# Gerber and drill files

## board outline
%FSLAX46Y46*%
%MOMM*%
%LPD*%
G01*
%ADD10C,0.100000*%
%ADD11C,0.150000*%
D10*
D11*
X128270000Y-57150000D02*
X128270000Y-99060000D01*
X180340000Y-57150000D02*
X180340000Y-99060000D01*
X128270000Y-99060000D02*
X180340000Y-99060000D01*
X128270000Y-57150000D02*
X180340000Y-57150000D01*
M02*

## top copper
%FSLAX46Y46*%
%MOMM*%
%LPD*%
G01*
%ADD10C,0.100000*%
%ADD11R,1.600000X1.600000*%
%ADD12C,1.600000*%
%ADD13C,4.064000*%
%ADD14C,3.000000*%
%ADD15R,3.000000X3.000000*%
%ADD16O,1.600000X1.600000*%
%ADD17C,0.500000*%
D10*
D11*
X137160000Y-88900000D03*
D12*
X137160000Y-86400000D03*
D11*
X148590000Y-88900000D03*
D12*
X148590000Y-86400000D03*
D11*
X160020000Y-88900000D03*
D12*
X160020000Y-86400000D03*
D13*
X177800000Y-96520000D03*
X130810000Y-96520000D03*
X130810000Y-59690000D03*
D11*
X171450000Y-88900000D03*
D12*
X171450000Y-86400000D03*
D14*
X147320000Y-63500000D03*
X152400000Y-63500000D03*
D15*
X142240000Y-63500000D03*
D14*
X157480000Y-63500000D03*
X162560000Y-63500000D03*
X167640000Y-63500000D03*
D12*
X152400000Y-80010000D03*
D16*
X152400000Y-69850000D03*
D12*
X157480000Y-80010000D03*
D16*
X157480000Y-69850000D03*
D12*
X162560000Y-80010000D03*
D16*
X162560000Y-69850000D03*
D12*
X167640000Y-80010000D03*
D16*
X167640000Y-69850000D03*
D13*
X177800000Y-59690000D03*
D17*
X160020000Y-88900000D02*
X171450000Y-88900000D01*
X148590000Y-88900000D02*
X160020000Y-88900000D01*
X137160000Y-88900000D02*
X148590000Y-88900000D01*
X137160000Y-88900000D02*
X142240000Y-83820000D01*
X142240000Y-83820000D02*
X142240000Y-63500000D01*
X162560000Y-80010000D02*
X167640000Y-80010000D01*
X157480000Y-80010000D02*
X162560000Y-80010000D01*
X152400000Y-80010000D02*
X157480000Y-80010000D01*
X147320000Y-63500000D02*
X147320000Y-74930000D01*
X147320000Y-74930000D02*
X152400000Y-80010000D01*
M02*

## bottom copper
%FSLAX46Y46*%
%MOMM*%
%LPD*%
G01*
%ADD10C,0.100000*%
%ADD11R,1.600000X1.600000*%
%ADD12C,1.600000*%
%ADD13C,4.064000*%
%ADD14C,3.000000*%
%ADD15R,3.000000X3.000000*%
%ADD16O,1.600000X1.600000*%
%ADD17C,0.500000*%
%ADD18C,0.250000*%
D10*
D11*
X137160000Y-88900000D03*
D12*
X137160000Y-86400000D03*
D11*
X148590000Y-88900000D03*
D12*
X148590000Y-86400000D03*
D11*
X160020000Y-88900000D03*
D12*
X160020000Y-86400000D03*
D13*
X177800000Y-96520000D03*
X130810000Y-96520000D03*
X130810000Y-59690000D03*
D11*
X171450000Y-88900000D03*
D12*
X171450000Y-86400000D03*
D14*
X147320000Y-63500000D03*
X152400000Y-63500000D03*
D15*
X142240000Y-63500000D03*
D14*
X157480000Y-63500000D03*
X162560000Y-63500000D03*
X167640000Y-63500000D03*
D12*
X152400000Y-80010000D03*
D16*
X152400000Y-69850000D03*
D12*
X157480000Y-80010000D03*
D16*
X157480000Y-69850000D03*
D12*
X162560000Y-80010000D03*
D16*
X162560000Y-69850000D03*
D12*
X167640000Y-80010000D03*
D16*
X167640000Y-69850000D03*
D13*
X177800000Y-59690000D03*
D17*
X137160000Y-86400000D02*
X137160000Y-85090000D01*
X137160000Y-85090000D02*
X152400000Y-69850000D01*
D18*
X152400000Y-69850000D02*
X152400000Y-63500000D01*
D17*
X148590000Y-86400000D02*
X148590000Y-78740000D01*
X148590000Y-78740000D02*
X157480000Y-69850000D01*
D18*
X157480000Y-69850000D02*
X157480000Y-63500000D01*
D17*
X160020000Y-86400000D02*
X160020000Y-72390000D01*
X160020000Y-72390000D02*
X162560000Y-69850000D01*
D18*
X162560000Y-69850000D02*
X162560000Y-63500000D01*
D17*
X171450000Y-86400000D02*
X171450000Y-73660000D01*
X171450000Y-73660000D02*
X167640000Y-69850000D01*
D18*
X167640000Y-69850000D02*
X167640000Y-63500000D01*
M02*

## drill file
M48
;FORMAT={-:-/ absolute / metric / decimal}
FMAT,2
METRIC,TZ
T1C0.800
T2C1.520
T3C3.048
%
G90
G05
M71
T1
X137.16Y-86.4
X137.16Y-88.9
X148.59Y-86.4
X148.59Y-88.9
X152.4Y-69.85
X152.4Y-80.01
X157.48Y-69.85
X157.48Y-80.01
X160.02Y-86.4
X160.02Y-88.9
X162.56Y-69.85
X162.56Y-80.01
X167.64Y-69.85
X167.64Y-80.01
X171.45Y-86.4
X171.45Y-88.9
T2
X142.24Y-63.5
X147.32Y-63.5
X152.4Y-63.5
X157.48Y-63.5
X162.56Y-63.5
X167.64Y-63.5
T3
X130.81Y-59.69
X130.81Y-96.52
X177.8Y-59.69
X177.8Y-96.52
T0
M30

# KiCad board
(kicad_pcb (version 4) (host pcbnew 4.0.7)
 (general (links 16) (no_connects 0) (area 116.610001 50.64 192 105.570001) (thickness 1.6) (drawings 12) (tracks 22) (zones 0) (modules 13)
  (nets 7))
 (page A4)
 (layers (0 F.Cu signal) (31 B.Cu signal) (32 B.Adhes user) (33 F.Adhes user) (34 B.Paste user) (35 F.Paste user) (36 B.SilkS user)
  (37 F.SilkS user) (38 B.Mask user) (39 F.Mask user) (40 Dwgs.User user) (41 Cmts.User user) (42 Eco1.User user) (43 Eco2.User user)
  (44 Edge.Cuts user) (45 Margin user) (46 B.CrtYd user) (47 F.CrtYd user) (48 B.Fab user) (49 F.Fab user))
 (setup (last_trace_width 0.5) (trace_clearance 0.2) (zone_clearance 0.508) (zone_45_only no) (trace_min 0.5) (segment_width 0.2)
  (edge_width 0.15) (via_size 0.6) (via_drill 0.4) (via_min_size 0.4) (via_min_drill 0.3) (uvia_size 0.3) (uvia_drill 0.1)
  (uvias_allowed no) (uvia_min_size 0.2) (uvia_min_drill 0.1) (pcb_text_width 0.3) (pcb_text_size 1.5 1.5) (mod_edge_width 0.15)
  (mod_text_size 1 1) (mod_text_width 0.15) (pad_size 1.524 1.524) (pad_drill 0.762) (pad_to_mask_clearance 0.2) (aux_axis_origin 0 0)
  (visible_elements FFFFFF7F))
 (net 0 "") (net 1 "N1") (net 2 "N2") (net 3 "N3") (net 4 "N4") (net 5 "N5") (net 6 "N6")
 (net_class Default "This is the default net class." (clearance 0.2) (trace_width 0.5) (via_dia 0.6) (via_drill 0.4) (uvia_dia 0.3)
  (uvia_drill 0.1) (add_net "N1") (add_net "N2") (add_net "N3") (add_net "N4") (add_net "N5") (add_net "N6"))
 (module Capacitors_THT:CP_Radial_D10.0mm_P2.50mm (layer F.Cu) (at 137.16 88.9 90)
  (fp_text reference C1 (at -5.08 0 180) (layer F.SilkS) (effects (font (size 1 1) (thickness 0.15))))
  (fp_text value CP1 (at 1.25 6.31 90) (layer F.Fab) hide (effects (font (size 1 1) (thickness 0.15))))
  (pad 1 thru_hole rect (at 0 0 90) (size 1.6 1.6) (drill 0.8) (layers *.Cu *.Mask) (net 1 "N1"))
  (pad 2 thru_hole circle (at 2.5 0 90) (size 1.6 1.6) (drill 0.8) (layers *.Cu *.Mask) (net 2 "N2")))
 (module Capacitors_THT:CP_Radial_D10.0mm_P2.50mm (layer F.Cu) (at 148.59 88.9 90)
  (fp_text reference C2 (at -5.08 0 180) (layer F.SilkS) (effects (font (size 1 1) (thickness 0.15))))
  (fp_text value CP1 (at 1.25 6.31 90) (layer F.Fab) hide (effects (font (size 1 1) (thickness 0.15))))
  (pad 1 thru_hole rect (at 0 0 90) (size 1.6 1.6) (drill 0.8) (layers *.Cu *.Mask) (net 1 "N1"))
  (pad 2 thru_hole circle (at 2.5 0 90) (size 1.6 1.6) (drill 0.8) (layers *.Cu *.Mask) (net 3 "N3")))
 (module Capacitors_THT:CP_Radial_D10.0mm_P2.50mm (layer F.Cu) (at 160.02 88.9 90)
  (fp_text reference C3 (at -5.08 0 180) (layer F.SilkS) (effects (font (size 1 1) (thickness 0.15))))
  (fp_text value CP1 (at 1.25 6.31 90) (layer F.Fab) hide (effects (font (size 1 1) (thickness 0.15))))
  (pad 1 thru_hole rect (at 0 0 90) (size 1.6 1.6) (drill 0.8) (layers *.Cu *.Mask) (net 1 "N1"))
  (pad 2 thru_hole circle (at 2.5 0 90) (size 1.6 1.6) (drill 0.8) (layers *.Cu *.Mask) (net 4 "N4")))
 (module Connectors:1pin (layer F.Cu) (at 177.8 96.52 180)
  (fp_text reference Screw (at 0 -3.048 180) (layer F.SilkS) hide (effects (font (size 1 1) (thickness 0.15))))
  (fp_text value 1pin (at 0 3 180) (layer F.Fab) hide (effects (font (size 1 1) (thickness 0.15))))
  (pad 1 thru_hole circle (at 0 0 180) (size 4.064 4.064) (drill 3.048) (layers *.Cu *.Mask)))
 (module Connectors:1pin (layer F.Cu) (at 130.81 96.52 180)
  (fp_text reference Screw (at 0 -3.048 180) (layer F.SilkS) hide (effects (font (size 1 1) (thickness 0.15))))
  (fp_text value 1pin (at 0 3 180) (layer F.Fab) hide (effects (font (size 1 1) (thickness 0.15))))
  (pad 1 thru_hole circle (at 0 0 180) (size 4.064 4.064) (drill 3.048) (layers *.Cu *.Mask)))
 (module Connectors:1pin (layer F.Cu) (at 130.81 59.69)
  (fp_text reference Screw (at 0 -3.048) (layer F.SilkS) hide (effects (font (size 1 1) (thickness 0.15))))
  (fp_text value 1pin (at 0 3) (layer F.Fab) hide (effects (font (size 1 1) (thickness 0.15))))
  (pad 1 thru_hole circle (at 0 0) (size 4.064 4.064) (drill 3.048) (layers *.Cu *.Mask)))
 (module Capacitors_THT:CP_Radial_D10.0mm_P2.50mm (layer F.Cu) (at 171.45 88.9 90)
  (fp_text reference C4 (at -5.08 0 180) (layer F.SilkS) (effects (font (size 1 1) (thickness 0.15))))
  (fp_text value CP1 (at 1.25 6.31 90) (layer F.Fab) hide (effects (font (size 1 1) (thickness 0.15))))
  (pad 1 thru_hole rect (at 0 0 90) (size 1.6 1.6) (drill 0.8) (layers *.Cu *.Mask) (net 1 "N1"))
  (pad 2 thru_hole circle (at 2.5 0 90) (size 1.6 1.6) (drill 0.8) (layers *.Cu *.Mask) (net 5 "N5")))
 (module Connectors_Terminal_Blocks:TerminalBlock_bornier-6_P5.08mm (layer F.Cu) (at 142.24 63.5)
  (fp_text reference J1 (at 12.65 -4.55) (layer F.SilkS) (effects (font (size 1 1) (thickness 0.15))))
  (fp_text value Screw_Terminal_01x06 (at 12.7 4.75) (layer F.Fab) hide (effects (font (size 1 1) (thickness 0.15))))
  (pad 2 thru_hole circle (at 5.08 0) (size 3 3) (drill 1.52) (layers *.Cu *.Mask) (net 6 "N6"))
  (pad 3 thru_hole circle (at 10.16 0) (size 3 3) (drill 1.52) (layers *.Cu *.Mask) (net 2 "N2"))
  (pad 1 thru_hole rect (at 0 0) (size 3 3) (drill 1.52) (layers *.Cu *.Mask) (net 1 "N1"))
  (pad 4 thru_hole circle (at 15.24 0) (size 3 3) (drill 1.52) (layers *.Cu *.Mask) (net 3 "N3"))
  (pad 5 thru_hole circle (at 20.32 0) (size 3 3) (drill 1.52) (layers *.Cu *.Mask) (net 4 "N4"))
  (pad 6 thru_hole circle (at 25.4 0) (size 3 3) (drill 1.52) (layers *.Cu *.Mask) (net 5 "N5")))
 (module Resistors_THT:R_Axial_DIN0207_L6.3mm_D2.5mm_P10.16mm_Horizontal (layer F.Cu) (at 152.4 80.01 90)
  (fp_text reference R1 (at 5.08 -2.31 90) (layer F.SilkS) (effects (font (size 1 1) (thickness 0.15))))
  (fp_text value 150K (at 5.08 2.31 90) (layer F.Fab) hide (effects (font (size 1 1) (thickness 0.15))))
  (pad 1 thru_hole circle (at 0 0 90) (size 1.6 1.6) (drill 0.8) (layers *.Cu *.Mask) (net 6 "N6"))
  (pad 2 thru_hole oval (at 10.16 0 90) (size 1.6 1.6) (drill 0.8) (layers *.Cu *.Mask) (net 2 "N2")))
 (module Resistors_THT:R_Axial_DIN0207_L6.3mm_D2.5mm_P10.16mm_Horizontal (layer F.Cu) (at 157.48 80.01 90)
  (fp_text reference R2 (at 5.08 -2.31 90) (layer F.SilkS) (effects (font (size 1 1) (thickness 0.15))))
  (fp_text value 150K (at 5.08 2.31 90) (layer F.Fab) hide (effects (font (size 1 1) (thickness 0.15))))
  (pad 1 thru_hole circle (at 0 0 90) (size 1.6 1.6) (drill 0.8) (layers *.Cu *.Mask) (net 6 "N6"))
  (pad 2 thru_hole oval (at 10.16 0 90) (size 1.6 1.6) (drill 0.8) (layers *.Cu *.Mask) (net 3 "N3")))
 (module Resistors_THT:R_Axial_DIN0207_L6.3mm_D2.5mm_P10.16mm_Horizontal (layer F.Cu) (at 162.56 80.01 90)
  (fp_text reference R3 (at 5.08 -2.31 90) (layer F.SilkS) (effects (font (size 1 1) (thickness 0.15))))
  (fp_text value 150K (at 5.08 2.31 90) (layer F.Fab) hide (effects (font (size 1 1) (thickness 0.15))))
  (pad 1 thru_hole circle (at 0 0 90) (size 1.6 1.6) (drill 0.8) (layers *.Cu *.Mask) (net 6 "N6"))
  (pad 2 thru_hole oval (at 10.16 0 90) (size 1.6 1.6) (drill 0.8) (layers *.Cu *.Mask) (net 4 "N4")))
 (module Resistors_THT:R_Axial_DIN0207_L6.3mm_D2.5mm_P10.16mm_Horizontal (layer F.Cu) (at 167.64 80.01 90)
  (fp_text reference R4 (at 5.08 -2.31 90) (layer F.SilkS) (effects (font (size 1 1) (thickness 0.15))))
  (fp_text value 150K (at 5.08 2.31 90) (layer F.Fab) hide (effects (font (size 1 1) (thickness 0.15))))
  (pad 1 thru_hole circle (at 0 0 90) (size 1.6 1.6) (drill 0.8) (layers *.Cu *.Mask) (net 6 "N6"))
  (pad 2 thru_hole oval (at 10.16 0 90) (size 1.6 1.6) (drill 0.8) (layers *.Cu *.Mask) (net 5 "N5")))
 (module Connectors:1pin (layer F.Cu) (at 177.8 59.69)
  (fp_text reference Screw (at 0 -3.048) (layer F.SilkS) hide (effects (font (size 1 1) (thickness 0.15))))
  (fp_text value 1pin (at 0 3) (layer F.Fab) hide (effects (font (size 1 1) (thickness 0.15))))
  (pad 1 thru_hole circle (at 0 0) (size 4.064 4.064) (drill 3.048) (layers *.Cu *.Mask)))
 (gr_line (start 128.27 57.15) (end 128.27 99.06) (angle 90) (layer Edge.Cuts) (width 0.15))
 (gr_line (start 180.34 57.15) (end 180.34 99.06) (angle 90) (layer Edge.Cuts) (width 0.15))
 (gr_line (start 128.27 99.06) (end 180.34 99.06) (angle 90) (layer Edge.Cuts) (width 0.15))
 (gr_line (start 128.27 57.15) (end 180.34 57.15) (angle 90) (layer Edge.Cuts) (width 0.15))
 (segment (start 160.02 88.9) (end 171.45 88.9) (width 0.5) (layer F.Cu) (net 1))
 (segment (start 148.59 88.9) (end 160.02 88.9) (width 0.5) (layer F.Cu) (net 1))
 (segment (start 137.16 88.9) (end 148.59 88.9) (width 0.5) (layer F.Cu) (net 1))
 (segment (start 137.16 88.9) (end 142.24 83.82) (width 0.5) (layer F.Cu) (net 1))
 (segment (start 142.24 83.82) (end 142.24 63.5) (width 0.5) (layer F.Cu) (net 1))
 (segment (start 137.16 86.4) (end 137.16 85.09) (width 0.5) (layer B.Cu) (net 2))
 (segment (start 137.16 85.09) (end 152.4 69.85) (width 0.5) (layer B.Cu) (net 2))
 (segment (start 152.4 69.85) (end 152.4 63.5) (width 0.25) (layer B.Cu) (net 2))
 (segment (start 148.59 86.4) (end 148.59 78.74) (width 0.5) (layer B.Cu) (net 3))
 (segment (start 148.59 78.74) (end 157.48 69.85) (width 0.5) (layer B.Cu) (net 3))
 (segment (start 157.48 69.85) (end 157.48 63.5) (width 0.25) (layer B.Cu) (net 3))
 (segment (start 160.02 86.4) (end 160.02 72.39) (width 0.5) (layer B.Cu) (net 4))
 (segment (start 160.02 72.39) (end 162.56 69.85) (width 0.5) (layer B.Cu) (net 4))
 (segment (start 162.56 69.85) (end 162.56 63.5) (width 0.25) (layer B.Cu) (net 4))
 (segment (start 171.45 86.4) (end 171.45 73.66) (width 0.5) (layer B.Cu) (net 5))
 (segment (start 171.45 73.66) (end 167.64 69.85) (width 0.5) (layer B.Cu) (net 5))
 (segment (start 167.64 69.85) (end 167.64 63.5) (width 0.25) (layer B.Cu) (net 5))
 (segment (start 162.56 80.01) (end 167.64 80.01) (width 0.5) (layer F.Cu) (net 6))
 (segment (start 157.48 80.01) (end 162.56 80.01) (width 0.5) (layer F.Cu) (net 6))
 (segment (start 152.4 80.01) (end 157.48 80.01) (width 0.5) (layer F.Cu) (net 6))
 (segment (start 147.32 63.5) (end 147.32 74.93) (width 0.5) (layer F.Cu) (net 6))
 (segment (start 147.32 74.93) (end 152.4 80.01) (width 0.5) (layer F.Cu) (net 6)))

